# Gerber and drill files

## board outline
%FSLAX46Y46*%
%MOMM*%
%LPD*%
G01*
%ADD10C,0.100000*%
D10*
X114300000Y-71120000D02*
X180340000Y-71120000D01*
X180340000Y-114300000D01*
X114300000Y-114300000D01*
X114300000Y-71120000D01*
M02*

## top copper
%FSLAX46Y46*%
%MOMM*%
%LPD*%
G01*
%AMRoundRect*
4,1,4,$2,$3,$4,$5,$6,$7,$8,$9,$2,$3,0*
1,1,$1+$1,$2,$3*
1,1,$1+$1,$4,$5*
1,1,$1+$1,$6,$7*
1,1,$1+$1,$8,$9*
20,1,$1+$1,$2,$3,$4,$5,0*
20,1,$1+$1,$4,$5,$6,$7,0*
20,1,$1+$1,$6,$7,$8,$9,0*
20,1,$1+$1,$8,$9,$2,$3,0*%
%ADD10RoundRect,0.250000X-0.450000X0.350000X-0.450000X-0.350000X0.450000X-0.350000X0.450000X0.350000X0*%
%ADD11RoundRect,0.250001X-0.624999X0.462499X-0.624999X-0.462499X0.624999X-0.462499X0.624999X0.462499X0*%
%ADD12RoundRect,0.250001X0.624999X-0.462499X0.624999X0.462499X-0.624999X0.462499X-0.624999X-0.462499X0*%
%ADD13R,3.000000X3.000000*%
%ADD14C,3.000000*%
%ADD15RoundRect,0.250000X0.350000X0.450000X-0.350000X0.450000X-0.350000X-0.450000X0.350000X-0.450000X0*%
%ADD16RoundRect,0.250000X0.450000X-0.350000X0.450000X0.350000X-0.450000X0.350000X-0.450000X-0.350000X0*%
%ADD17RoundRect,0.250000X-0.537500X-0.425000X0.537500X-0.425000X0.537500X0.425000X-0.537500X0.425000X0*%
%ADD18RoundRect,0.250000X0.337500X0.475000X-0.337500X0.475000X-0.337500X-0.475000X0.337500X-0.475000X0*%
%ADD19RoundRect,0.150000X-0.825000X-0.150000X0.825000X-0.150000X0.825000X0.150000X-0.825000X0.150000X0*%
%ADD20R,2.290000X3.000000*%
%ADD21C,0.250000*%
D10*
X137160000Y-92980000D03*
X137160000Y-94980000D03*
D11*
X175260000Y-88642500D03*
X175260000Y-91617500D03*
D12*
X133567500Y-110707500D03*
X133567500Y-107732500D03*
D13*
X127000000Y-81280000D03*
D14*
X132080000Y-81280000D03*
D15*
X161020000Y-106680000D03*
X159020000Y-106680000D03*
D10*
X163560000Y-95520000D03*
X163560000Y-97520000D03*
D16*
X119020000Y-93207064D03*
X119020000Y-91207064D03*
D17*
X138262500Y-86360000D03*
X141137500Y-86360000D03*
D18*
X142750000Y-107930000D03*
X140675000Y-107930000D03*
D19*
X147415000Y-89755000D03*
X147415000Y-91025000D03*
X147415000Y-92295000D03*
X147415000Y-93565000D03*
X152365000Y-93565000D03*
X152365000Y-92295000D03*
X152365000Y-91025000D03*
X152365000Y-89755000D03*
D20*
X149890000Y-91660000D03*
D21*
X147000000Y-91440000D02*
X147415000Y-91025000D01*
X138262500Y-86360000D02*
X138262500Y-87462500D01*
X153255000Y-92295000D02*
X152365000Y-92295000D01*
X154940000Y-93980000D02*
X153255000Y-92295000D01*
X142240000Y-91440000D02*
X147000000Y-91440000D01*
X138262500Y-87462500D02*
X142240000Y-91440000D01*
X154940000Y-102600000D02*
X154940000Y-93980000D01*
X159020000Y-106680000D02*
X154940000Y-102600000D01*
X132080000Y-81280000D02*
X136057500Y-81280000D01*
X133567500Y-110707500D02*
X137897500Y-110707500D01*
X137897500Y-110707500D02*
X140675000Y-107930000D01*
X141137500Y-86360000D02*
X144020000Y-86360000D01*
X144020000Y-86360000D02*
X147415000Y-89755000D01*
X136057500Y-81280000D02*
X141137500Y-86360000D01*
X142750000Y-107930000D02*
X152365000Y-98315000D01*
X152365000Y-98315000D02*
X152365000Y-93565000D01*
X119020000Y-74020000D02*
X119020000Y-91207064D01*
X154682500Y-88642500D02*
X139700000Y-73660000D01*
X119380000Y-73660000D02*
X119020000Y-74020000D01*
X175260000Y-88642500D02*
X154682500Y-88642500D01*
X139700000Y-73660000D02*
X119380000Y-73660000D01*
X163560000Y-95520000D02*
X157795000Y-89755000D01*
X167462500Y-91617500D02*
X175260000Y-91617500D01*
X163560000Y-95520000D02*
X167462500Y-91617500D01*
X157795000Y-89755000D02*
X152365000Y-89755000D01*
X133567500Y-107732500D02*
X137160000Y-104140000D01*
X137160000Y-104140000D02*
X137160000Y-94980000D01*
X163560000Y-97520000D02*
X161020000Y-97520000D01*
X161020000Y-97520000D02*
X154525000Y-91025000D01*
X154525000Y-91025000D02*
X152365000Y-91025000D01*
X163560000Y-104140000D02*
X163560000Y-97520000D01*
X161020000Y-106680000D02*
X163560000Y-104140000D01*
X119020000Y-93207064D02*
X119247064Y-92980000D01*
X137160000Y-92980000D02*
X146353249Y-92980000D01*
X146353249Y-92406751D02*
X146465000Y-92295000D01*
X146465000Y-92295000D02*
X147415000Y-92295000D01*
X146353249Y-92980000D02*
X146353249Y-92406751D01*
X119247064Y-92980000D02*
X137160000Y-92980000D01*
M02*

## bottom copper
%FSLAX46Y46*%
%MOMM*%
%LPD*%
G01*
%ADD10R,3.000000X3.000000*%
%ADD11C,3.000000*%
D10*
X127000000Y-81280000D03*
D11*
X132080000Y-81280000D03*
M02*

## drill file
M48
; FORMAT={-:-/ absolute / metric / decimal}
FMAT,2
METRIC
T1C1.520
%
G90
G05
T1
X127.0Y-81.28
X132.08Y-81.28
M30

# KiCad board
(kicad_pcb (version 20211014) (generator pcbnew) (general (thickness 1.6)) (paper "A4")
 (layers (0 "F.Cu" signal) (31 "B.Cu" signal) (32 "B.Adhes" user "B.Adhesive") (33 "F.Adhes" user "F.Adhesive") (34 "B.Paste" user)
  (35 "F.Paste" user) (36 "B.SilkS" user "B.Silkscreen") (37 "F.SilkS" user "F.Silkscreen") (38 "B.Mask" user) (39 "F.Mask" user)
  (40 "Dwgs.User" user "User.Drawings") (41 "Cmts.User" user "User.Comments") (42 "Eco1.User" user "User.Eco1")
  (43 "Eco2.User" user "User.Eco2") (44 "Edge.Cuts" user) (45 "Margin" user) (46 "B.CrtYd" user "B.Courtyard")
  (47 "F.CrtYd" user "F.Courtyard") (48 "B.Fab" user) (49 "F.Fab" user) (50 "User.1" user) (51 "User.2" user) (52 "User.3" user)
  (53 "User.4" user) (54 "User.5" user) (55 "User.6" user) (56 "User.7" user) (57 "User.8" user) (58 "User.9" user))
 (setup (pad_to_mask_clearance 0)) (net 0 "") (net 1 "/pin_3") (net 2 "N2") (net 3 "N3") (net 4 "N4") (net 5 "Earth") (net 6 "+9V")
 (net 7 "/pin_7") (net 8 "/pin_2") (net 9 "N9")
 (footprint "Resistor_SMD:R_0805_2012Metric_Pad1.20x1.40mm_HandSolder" (layer "F.Cu") (at 137.16 93.98 -90)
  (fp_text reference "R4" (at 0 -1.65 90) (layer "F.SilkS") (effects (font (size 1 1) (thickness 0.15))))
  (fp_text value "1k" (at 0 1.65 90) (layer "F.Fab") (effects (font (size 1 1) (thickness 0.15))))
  (pad "1" smd roundrect (at -1 0 270) (size 1.2 1.4) (layers "F.Cu" "F.Paste" "F.Mask") (roundrect_rratio 0.2083333333) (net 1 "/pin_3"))
  (pad "2" smd roundrect (at 1 0 270) (size 1.2 1.4) (layers "F.Cu" "F.Paste" "F.Mask") (roundrect_rratio 0.2083333333) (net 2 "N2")))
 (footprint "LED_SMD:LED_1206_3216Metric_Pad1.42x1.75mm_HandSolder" (layer "F.Cu") (at 175.26 90.13 -90)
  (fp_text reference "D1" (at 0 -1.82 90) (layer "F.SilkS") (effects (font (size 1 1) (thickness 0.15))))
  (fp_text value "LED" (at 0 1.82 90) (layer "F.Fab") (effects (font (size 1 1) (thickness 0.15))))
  (pad "1" smd roundrect (at -1.4875 0 270) (size 1.425 1.75) (layers "F.Cu" "F.Paste" "F.Mask") (roundrect_rratio 0.1754392982)
   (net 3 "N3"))
  (pad "2" smd roundrect (at 1.4875 0 270) (size 1.425 1.75) (layers "F.Cu" "F.Paste" "F.Mask") (roundrect_rratio 0.1754392982) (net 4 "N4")))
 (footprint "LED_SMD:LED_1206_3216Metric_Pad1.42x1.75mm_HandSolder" (layer "F.Cu") (at 133.5675 109.22 90)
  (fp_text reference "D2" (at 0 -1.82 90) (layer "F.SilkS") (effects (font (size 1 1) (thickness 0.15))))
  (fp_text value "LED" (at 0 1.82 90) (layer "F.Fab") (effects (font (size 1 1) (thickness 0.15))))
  (pad "1" smd roundrect (at -1.4875 0 90) (size 1.425 1.75) (layers "F.Cu" "F.Paste" "F.Mask") (roundrect_rratio 0.1754392982)
   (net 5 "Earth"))
  (pad "2" smd roundrect (at 1.4875 0 90) (size 1.425 1.75) (layers "F.Cu" "F.Paste" "F.Mask") (roundrect_rratio 0.1754392982) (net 2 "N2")))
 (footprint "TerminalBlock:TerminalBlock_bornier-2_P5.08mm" (layer "F.Cu") (at 127 81.28)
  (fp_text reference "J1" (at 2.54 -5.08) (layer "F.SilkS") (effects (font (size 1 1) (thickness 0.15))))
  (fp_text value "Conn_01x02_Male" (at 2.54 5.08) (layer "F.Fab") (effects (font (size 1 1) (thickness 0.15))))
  (pad "1" thru_hole rect (at 0 0) (size 3 3) (drill 1.52) (layers *.Cu *.Mask) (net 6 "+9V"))
  (pad "2" thru_hole circle (at 5.08 0) (size 3 3) (drill 1.52) (layers *.Cu *.Mask) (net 5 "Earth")))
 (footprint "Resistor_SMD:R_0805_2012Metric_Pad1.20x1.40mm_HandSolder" (layer "F.Cu") (at 160.02 106.68 180)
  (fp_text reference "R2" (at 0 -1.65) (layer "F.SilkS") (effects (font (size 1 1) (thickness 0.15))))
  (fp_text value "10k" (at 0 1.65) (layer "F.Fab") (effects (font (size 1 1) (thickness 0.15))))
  (pad "1" smd roundrect (at -1 0 180) (size 1.2 1.4) (layers "F.Cu" "F.Paste" "F.Mask") (roundrect_rratio 0.2083333333) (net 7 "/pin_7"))
  (pad "2" smd roundrect (at 1 0 180) (size 1.2 1.4) (layers "F.Cu" "F.Paste" "F.Mask") (roundrect_rratio 0.2083333333) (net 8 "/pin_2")))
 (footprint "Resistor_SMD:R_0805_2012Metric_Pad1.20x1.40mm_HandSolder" (layer "F.Cu") (at 163.56 96.52 -90)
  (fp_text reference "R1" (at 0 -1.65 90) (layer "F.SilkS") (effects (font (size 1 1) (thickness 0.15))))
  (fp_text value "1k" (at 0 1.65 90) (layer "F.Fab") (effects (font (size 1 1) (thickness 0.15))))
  (pad "1" smd roundrect (at -1 0 270) (size 1.2 1.4) (layers "F.Cu" "F.Paste" "F.Mask") (roundrect_rratio 0.2083333333) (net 4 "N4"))
  (pad "2" smd roundrect (at 1 0 270) (size 1.2 1.4) (layers "F.Cu" "F.Paste" "F.Mask") (roundrect_rratio 0.2083333333) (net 7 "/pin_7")))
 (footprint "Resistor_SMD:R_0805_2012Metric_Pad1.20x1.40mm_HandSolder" (layer "F.Cu") (at 119.02 92.207064 90)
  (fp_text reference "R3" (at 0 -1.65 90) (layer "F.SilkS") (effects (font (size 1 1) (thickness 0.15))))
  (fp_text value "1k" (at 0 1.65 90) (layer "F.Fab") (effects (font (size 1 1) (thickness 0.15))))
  (pad "1" smd roundrect (at -1 0 90) (size 1.2 1.4) (layers "F.Cu" "F.Paste" "F.Mask") (roundrect_rratio 0.2083333333) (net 1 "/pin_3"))
  (pad "2" smd roundrect (at 1 0 90) (size 1.2 1.4) (layers "F.Cu" "F.Paste" "F.Mask") (roundrect_rratio 0.2083333333) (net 3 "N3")))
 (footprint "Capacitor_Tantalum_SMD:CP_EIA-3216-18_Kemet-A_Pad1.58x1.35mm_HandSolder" (layer "F.Cu") (at 139.7 86.36)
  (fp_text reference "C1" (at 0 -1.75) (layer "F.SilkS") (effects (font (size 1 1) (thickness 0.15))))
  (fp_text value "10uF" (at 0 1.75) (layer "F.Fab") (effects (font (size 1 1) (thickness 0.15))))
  (pad "1" smd roundrect (at -1.4375 0) (size 1.575 1.35) (layers "F.Cu" "F.Paste" "F.Mask") (roundrect_rratio 0.1851851852)
   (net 8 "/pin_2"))
  (pad "2" smd roundrect (at 1.4375 0) (size 1.575 1.35) (layers "F.Cu" "F.Paste" "F.Mask") (roundrect_rratio 0.1851851852) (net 5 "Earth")))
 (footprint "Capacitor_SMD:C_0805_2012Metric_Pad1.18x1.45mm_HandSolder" (layer "F.Cu") (at 141.7125 107.93 180)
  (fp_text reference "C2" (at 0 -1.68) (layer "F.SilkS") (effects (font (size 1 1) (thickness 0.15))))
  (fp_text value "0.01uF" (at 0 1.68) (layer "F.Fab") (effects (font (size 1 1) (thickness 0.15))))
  (pad "1" smd roundrect (at -1.0375 0 180) (size 1.175 1.45) (layers "F.Cu" "F.Paste" "F.Mask") (roundrect_rratio 0.2127659574)
   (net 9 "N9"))
  (pad "2" smd roundrect (at 1.0375 0 180) (size 1.175 1.45) (layers "F.Cu" "F.Paste" "F.Mask") (roundrect_rratio 0.2127659574)
   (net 5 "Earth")))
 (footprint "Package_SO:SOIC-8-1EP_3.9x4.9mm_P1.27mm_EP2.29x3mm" (layer "F.Cu") (at 149.89 91.66)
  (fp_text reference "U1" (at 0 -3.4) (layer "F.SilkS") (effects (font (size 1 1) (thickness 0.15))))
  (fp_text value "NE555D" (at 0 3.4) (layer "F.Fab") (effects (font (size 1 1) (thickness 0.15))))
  (pad "" smd roundrect (at -0.57 0.75) (size 0.92 1.21) (layers "F.Paste") (roundrect_rratio 0.25))
  (pad "" smd roundrect (at 0.57 -0.75) (size 0.92 1.21) (layers "F.Paste") (roundrect_rratio 0.25))
  (pad "" smd roundrect (at 0.57 0.75) (size 0.92 1.21) (layers "F.Paste") (roundrect_rratio 0.25))
  (pad "" smd roundrect (at -0.57 -0.75) (size 0.92 1.21) (layers "F.Paste") (roundrect_rratio 0.25))
  (pad "1" smd roundrect (at -2.475 -1.905) (size 1.95 0.6) (layers "F.Cu" "F.Paste" "F.Mask") (roundrect_rratio 0.25) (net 5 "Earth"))
  (pad "2" smd roundrect (at -2.475 -0.635) (size 1.95 0.6) (layers "F.Cu" "F.Paste" "F.Mask") (roundrect_rratio 0.25) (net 8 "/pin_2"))
  (pad "3" smd roundrect (at -2.475 0.635) (size 1.95 0.6) (layers "F.Cu" "F.Paste" "F.Mask") (roundrect_rratio 0.25) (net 1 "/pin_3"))
  (pad "4" smd roundrect (at -2.475 1.905) (size 1.95 0.6) (layers "F.Cu" "F.Paste" "F.Mask") (roundrect_rratio 0.25) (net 4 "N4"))
  (pad "5" smd roundrect (at 2.475 1.905) (size 1.95 0.6) (layers "F.Cu" "F.Paste" "F.Mask") (roundrect_rratio 0.25) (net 9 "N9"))
  (pad "6" smd roundrect (at 2.475 0.635) (size 1.95 0.6) (layers "F.Cu" "F.Paste" "F.Mask") (roundrect_rratio 0.25) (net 8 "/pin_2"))
  (pad "7" smd roundrect (at 2.475 -0.635) (size 1.95 0.6) (layers "F.Cu" "F.Paste" "F.Mask") (roundrect_rratio 0.25) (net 7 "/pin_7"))
  (pad "8" smd roundrect (at 2.475 -1.905) (size 1.95 0.6) (layers "F.Cu" "F.Paste" "F.Mask") (roundrect_rratio 0.25) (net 4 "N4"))
  (pad "9" smd rect (at 0 0) (size 2.29 3) (layers "F.Cu" "F.Mask")))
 (gr_rect (start 114.3 71.12) (end 180.34 114.3) (layer "Edge.Cuts") (width 0.1) (fill none))
 (segment (start 147 91.44) (end 147.415 91.025) (width 0.25) (layer "F.Cu") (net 8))
 (segment (start 138.2625 86.36) (end 138.2625 87.4625) (width 0.25) (layer "F.Cu") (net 8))
 (segment (start 153.255 92.295) (end 152.365 92.295) (width 0.25) (layer "F.Cu") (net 8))
 (segment (start 154.94 93.98) (end 153.255 92.295) (width 0.25) (layer "F.Cu") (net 8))
 (segment (start 142.24 91.44) (end 147 91.44) (width 0.25) (layer "F.Cu") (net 8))
 (segment (start 138.2625 87.4625) (end 142.24 91.44) (width 0.25) (layer "F.Cu") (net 8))
 (segment (start 154.94 102.6) (end 154.94 93.98) (width 0.25) (layer "F.Cu") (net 8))
 (segment (start 159.02 106.68) (end 154.94 102.6) (width 0.25) (layer "F.Cu") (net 8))
 (segment (start 132.08 81.28) (end 136.0575 81.28) (width 0.25) (layer "F.Cu") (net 5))
 (segment (start 133.5675 110.7075) (end 137.8975 110.7075) (width 0.25) (layer "F.Cu") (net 5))
 (segment (start 137.8975 110.7075) (end 140.675 107.93) (width 0.25) (layer "F.Cu") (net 5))
 (segment (start 141.1375 86.36) (end 144.02 86.36) (width 0.25) (layer "F.Cu") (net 5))
 (segment (start 144.02 86.36) (end 147.415 89.755) (width 0.25) (layer "F.Cu") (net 5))
 (segment (start 136.0575 81.28) (end 141.1375 86.36) (width 0.25) (layer "F.Cu") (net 5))
 (segment (start 142.75 107.93) (end 152.365 98.315) (width 0.25) (layer "F.Cu") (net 9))
 (segment (start 152.365 98.315) (end 152.365 93.565) (width 0.25) (layer "F.Cu") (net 9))
 (segment (start 119.02 74.02) (end 119.02 91.207064) (width 0.25) (layer "F.Cu") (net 3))
 (segment (start 154.6825 88.6425) (end 139.7 73.66) (width 0.25) (layer "F.Cu") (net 3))
 (segment (start 119.38 73.66) (end 119.02 74.02) (width 0.25) (layer "F.Cu") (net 3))
 (segment (start 175.26 88.6425) (end 154.6825 88.6425) (width 0.25) (layer "F.Cu") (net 3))
 (segment (start 139.7 73.66) (end 119.38 73.66) (width 0.25) (layer "F.Cu") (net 3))
 (segment (start 163.56 95.52) (end 157.795 89.755) (width 0.25) (layer "F.Cu") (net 4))
 (segment (start 167.4625 91.6175) (end 175.26 91.6175) (width 0.25) (layer "F.Cu") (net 4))
 (segment (start 163.56 95.52) (end 167.4625 91.6175) (width 0.25) (layer "F.Cu") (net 4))
 (segment (start 157.795 89.755) (end 152.365 89.755) (width 0.25) (layer "F.Cu") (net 4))
 (segment (start 133.5675 107.7325) (end 137.16 104.14) (width 0.25) (layer "F.Cu") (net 2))
 (segment (start 137.16 104.14) (end 137.16 94.98) (width 0.25) (layer "F.Cu") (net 2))
 (segment (start 163.56 97.52) (end 161.02 97.52) (width 0.25) (layer "F.Cu") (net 7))
 (segment (start 161.02 97.52) (end 154.525 91.025) (width 0.25) (layer "F.Cu") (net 7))
 (segment (start 154.525 91.025) (end 152.365 91.025) (width 0.25) (layer "F.Cu") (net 7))
 (segment (start 163.56 104.14) (end 163.56 97.52) (width 0.25) (layer "F.Cu") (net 7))
 (segment (start 161.02 106.68) (end 163.56 104.14) (width 0.25) (layer "F.Cu") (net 7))
 (segment (start 119.02 93.207064) (end 119.247064 92.98) (width 0.25) (layer "F.Cu") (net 1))
 (segment (start 137.16 92.98) (end 146.353249 92.98) (width 0.25) (layer "F.Cu") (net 1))
 (segment (start 146.353249 92.406751) (end 146.465 92.295) (width 0.25) (layer "F.Cu") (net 1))
 (segment (start 146.465 92.295) (end 147.415 92.295) (width 0.25) (layer "F.Cu") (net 1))
 (segment (start 146.353249 92.98) (end 146.353249 92.406751) (width 0.25) (layer "F.Cu") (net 1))
 (segment (start 119.247064 92.98) (end 137.16 92.98) (width 0.25) (layer "F.Cu") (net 1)))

